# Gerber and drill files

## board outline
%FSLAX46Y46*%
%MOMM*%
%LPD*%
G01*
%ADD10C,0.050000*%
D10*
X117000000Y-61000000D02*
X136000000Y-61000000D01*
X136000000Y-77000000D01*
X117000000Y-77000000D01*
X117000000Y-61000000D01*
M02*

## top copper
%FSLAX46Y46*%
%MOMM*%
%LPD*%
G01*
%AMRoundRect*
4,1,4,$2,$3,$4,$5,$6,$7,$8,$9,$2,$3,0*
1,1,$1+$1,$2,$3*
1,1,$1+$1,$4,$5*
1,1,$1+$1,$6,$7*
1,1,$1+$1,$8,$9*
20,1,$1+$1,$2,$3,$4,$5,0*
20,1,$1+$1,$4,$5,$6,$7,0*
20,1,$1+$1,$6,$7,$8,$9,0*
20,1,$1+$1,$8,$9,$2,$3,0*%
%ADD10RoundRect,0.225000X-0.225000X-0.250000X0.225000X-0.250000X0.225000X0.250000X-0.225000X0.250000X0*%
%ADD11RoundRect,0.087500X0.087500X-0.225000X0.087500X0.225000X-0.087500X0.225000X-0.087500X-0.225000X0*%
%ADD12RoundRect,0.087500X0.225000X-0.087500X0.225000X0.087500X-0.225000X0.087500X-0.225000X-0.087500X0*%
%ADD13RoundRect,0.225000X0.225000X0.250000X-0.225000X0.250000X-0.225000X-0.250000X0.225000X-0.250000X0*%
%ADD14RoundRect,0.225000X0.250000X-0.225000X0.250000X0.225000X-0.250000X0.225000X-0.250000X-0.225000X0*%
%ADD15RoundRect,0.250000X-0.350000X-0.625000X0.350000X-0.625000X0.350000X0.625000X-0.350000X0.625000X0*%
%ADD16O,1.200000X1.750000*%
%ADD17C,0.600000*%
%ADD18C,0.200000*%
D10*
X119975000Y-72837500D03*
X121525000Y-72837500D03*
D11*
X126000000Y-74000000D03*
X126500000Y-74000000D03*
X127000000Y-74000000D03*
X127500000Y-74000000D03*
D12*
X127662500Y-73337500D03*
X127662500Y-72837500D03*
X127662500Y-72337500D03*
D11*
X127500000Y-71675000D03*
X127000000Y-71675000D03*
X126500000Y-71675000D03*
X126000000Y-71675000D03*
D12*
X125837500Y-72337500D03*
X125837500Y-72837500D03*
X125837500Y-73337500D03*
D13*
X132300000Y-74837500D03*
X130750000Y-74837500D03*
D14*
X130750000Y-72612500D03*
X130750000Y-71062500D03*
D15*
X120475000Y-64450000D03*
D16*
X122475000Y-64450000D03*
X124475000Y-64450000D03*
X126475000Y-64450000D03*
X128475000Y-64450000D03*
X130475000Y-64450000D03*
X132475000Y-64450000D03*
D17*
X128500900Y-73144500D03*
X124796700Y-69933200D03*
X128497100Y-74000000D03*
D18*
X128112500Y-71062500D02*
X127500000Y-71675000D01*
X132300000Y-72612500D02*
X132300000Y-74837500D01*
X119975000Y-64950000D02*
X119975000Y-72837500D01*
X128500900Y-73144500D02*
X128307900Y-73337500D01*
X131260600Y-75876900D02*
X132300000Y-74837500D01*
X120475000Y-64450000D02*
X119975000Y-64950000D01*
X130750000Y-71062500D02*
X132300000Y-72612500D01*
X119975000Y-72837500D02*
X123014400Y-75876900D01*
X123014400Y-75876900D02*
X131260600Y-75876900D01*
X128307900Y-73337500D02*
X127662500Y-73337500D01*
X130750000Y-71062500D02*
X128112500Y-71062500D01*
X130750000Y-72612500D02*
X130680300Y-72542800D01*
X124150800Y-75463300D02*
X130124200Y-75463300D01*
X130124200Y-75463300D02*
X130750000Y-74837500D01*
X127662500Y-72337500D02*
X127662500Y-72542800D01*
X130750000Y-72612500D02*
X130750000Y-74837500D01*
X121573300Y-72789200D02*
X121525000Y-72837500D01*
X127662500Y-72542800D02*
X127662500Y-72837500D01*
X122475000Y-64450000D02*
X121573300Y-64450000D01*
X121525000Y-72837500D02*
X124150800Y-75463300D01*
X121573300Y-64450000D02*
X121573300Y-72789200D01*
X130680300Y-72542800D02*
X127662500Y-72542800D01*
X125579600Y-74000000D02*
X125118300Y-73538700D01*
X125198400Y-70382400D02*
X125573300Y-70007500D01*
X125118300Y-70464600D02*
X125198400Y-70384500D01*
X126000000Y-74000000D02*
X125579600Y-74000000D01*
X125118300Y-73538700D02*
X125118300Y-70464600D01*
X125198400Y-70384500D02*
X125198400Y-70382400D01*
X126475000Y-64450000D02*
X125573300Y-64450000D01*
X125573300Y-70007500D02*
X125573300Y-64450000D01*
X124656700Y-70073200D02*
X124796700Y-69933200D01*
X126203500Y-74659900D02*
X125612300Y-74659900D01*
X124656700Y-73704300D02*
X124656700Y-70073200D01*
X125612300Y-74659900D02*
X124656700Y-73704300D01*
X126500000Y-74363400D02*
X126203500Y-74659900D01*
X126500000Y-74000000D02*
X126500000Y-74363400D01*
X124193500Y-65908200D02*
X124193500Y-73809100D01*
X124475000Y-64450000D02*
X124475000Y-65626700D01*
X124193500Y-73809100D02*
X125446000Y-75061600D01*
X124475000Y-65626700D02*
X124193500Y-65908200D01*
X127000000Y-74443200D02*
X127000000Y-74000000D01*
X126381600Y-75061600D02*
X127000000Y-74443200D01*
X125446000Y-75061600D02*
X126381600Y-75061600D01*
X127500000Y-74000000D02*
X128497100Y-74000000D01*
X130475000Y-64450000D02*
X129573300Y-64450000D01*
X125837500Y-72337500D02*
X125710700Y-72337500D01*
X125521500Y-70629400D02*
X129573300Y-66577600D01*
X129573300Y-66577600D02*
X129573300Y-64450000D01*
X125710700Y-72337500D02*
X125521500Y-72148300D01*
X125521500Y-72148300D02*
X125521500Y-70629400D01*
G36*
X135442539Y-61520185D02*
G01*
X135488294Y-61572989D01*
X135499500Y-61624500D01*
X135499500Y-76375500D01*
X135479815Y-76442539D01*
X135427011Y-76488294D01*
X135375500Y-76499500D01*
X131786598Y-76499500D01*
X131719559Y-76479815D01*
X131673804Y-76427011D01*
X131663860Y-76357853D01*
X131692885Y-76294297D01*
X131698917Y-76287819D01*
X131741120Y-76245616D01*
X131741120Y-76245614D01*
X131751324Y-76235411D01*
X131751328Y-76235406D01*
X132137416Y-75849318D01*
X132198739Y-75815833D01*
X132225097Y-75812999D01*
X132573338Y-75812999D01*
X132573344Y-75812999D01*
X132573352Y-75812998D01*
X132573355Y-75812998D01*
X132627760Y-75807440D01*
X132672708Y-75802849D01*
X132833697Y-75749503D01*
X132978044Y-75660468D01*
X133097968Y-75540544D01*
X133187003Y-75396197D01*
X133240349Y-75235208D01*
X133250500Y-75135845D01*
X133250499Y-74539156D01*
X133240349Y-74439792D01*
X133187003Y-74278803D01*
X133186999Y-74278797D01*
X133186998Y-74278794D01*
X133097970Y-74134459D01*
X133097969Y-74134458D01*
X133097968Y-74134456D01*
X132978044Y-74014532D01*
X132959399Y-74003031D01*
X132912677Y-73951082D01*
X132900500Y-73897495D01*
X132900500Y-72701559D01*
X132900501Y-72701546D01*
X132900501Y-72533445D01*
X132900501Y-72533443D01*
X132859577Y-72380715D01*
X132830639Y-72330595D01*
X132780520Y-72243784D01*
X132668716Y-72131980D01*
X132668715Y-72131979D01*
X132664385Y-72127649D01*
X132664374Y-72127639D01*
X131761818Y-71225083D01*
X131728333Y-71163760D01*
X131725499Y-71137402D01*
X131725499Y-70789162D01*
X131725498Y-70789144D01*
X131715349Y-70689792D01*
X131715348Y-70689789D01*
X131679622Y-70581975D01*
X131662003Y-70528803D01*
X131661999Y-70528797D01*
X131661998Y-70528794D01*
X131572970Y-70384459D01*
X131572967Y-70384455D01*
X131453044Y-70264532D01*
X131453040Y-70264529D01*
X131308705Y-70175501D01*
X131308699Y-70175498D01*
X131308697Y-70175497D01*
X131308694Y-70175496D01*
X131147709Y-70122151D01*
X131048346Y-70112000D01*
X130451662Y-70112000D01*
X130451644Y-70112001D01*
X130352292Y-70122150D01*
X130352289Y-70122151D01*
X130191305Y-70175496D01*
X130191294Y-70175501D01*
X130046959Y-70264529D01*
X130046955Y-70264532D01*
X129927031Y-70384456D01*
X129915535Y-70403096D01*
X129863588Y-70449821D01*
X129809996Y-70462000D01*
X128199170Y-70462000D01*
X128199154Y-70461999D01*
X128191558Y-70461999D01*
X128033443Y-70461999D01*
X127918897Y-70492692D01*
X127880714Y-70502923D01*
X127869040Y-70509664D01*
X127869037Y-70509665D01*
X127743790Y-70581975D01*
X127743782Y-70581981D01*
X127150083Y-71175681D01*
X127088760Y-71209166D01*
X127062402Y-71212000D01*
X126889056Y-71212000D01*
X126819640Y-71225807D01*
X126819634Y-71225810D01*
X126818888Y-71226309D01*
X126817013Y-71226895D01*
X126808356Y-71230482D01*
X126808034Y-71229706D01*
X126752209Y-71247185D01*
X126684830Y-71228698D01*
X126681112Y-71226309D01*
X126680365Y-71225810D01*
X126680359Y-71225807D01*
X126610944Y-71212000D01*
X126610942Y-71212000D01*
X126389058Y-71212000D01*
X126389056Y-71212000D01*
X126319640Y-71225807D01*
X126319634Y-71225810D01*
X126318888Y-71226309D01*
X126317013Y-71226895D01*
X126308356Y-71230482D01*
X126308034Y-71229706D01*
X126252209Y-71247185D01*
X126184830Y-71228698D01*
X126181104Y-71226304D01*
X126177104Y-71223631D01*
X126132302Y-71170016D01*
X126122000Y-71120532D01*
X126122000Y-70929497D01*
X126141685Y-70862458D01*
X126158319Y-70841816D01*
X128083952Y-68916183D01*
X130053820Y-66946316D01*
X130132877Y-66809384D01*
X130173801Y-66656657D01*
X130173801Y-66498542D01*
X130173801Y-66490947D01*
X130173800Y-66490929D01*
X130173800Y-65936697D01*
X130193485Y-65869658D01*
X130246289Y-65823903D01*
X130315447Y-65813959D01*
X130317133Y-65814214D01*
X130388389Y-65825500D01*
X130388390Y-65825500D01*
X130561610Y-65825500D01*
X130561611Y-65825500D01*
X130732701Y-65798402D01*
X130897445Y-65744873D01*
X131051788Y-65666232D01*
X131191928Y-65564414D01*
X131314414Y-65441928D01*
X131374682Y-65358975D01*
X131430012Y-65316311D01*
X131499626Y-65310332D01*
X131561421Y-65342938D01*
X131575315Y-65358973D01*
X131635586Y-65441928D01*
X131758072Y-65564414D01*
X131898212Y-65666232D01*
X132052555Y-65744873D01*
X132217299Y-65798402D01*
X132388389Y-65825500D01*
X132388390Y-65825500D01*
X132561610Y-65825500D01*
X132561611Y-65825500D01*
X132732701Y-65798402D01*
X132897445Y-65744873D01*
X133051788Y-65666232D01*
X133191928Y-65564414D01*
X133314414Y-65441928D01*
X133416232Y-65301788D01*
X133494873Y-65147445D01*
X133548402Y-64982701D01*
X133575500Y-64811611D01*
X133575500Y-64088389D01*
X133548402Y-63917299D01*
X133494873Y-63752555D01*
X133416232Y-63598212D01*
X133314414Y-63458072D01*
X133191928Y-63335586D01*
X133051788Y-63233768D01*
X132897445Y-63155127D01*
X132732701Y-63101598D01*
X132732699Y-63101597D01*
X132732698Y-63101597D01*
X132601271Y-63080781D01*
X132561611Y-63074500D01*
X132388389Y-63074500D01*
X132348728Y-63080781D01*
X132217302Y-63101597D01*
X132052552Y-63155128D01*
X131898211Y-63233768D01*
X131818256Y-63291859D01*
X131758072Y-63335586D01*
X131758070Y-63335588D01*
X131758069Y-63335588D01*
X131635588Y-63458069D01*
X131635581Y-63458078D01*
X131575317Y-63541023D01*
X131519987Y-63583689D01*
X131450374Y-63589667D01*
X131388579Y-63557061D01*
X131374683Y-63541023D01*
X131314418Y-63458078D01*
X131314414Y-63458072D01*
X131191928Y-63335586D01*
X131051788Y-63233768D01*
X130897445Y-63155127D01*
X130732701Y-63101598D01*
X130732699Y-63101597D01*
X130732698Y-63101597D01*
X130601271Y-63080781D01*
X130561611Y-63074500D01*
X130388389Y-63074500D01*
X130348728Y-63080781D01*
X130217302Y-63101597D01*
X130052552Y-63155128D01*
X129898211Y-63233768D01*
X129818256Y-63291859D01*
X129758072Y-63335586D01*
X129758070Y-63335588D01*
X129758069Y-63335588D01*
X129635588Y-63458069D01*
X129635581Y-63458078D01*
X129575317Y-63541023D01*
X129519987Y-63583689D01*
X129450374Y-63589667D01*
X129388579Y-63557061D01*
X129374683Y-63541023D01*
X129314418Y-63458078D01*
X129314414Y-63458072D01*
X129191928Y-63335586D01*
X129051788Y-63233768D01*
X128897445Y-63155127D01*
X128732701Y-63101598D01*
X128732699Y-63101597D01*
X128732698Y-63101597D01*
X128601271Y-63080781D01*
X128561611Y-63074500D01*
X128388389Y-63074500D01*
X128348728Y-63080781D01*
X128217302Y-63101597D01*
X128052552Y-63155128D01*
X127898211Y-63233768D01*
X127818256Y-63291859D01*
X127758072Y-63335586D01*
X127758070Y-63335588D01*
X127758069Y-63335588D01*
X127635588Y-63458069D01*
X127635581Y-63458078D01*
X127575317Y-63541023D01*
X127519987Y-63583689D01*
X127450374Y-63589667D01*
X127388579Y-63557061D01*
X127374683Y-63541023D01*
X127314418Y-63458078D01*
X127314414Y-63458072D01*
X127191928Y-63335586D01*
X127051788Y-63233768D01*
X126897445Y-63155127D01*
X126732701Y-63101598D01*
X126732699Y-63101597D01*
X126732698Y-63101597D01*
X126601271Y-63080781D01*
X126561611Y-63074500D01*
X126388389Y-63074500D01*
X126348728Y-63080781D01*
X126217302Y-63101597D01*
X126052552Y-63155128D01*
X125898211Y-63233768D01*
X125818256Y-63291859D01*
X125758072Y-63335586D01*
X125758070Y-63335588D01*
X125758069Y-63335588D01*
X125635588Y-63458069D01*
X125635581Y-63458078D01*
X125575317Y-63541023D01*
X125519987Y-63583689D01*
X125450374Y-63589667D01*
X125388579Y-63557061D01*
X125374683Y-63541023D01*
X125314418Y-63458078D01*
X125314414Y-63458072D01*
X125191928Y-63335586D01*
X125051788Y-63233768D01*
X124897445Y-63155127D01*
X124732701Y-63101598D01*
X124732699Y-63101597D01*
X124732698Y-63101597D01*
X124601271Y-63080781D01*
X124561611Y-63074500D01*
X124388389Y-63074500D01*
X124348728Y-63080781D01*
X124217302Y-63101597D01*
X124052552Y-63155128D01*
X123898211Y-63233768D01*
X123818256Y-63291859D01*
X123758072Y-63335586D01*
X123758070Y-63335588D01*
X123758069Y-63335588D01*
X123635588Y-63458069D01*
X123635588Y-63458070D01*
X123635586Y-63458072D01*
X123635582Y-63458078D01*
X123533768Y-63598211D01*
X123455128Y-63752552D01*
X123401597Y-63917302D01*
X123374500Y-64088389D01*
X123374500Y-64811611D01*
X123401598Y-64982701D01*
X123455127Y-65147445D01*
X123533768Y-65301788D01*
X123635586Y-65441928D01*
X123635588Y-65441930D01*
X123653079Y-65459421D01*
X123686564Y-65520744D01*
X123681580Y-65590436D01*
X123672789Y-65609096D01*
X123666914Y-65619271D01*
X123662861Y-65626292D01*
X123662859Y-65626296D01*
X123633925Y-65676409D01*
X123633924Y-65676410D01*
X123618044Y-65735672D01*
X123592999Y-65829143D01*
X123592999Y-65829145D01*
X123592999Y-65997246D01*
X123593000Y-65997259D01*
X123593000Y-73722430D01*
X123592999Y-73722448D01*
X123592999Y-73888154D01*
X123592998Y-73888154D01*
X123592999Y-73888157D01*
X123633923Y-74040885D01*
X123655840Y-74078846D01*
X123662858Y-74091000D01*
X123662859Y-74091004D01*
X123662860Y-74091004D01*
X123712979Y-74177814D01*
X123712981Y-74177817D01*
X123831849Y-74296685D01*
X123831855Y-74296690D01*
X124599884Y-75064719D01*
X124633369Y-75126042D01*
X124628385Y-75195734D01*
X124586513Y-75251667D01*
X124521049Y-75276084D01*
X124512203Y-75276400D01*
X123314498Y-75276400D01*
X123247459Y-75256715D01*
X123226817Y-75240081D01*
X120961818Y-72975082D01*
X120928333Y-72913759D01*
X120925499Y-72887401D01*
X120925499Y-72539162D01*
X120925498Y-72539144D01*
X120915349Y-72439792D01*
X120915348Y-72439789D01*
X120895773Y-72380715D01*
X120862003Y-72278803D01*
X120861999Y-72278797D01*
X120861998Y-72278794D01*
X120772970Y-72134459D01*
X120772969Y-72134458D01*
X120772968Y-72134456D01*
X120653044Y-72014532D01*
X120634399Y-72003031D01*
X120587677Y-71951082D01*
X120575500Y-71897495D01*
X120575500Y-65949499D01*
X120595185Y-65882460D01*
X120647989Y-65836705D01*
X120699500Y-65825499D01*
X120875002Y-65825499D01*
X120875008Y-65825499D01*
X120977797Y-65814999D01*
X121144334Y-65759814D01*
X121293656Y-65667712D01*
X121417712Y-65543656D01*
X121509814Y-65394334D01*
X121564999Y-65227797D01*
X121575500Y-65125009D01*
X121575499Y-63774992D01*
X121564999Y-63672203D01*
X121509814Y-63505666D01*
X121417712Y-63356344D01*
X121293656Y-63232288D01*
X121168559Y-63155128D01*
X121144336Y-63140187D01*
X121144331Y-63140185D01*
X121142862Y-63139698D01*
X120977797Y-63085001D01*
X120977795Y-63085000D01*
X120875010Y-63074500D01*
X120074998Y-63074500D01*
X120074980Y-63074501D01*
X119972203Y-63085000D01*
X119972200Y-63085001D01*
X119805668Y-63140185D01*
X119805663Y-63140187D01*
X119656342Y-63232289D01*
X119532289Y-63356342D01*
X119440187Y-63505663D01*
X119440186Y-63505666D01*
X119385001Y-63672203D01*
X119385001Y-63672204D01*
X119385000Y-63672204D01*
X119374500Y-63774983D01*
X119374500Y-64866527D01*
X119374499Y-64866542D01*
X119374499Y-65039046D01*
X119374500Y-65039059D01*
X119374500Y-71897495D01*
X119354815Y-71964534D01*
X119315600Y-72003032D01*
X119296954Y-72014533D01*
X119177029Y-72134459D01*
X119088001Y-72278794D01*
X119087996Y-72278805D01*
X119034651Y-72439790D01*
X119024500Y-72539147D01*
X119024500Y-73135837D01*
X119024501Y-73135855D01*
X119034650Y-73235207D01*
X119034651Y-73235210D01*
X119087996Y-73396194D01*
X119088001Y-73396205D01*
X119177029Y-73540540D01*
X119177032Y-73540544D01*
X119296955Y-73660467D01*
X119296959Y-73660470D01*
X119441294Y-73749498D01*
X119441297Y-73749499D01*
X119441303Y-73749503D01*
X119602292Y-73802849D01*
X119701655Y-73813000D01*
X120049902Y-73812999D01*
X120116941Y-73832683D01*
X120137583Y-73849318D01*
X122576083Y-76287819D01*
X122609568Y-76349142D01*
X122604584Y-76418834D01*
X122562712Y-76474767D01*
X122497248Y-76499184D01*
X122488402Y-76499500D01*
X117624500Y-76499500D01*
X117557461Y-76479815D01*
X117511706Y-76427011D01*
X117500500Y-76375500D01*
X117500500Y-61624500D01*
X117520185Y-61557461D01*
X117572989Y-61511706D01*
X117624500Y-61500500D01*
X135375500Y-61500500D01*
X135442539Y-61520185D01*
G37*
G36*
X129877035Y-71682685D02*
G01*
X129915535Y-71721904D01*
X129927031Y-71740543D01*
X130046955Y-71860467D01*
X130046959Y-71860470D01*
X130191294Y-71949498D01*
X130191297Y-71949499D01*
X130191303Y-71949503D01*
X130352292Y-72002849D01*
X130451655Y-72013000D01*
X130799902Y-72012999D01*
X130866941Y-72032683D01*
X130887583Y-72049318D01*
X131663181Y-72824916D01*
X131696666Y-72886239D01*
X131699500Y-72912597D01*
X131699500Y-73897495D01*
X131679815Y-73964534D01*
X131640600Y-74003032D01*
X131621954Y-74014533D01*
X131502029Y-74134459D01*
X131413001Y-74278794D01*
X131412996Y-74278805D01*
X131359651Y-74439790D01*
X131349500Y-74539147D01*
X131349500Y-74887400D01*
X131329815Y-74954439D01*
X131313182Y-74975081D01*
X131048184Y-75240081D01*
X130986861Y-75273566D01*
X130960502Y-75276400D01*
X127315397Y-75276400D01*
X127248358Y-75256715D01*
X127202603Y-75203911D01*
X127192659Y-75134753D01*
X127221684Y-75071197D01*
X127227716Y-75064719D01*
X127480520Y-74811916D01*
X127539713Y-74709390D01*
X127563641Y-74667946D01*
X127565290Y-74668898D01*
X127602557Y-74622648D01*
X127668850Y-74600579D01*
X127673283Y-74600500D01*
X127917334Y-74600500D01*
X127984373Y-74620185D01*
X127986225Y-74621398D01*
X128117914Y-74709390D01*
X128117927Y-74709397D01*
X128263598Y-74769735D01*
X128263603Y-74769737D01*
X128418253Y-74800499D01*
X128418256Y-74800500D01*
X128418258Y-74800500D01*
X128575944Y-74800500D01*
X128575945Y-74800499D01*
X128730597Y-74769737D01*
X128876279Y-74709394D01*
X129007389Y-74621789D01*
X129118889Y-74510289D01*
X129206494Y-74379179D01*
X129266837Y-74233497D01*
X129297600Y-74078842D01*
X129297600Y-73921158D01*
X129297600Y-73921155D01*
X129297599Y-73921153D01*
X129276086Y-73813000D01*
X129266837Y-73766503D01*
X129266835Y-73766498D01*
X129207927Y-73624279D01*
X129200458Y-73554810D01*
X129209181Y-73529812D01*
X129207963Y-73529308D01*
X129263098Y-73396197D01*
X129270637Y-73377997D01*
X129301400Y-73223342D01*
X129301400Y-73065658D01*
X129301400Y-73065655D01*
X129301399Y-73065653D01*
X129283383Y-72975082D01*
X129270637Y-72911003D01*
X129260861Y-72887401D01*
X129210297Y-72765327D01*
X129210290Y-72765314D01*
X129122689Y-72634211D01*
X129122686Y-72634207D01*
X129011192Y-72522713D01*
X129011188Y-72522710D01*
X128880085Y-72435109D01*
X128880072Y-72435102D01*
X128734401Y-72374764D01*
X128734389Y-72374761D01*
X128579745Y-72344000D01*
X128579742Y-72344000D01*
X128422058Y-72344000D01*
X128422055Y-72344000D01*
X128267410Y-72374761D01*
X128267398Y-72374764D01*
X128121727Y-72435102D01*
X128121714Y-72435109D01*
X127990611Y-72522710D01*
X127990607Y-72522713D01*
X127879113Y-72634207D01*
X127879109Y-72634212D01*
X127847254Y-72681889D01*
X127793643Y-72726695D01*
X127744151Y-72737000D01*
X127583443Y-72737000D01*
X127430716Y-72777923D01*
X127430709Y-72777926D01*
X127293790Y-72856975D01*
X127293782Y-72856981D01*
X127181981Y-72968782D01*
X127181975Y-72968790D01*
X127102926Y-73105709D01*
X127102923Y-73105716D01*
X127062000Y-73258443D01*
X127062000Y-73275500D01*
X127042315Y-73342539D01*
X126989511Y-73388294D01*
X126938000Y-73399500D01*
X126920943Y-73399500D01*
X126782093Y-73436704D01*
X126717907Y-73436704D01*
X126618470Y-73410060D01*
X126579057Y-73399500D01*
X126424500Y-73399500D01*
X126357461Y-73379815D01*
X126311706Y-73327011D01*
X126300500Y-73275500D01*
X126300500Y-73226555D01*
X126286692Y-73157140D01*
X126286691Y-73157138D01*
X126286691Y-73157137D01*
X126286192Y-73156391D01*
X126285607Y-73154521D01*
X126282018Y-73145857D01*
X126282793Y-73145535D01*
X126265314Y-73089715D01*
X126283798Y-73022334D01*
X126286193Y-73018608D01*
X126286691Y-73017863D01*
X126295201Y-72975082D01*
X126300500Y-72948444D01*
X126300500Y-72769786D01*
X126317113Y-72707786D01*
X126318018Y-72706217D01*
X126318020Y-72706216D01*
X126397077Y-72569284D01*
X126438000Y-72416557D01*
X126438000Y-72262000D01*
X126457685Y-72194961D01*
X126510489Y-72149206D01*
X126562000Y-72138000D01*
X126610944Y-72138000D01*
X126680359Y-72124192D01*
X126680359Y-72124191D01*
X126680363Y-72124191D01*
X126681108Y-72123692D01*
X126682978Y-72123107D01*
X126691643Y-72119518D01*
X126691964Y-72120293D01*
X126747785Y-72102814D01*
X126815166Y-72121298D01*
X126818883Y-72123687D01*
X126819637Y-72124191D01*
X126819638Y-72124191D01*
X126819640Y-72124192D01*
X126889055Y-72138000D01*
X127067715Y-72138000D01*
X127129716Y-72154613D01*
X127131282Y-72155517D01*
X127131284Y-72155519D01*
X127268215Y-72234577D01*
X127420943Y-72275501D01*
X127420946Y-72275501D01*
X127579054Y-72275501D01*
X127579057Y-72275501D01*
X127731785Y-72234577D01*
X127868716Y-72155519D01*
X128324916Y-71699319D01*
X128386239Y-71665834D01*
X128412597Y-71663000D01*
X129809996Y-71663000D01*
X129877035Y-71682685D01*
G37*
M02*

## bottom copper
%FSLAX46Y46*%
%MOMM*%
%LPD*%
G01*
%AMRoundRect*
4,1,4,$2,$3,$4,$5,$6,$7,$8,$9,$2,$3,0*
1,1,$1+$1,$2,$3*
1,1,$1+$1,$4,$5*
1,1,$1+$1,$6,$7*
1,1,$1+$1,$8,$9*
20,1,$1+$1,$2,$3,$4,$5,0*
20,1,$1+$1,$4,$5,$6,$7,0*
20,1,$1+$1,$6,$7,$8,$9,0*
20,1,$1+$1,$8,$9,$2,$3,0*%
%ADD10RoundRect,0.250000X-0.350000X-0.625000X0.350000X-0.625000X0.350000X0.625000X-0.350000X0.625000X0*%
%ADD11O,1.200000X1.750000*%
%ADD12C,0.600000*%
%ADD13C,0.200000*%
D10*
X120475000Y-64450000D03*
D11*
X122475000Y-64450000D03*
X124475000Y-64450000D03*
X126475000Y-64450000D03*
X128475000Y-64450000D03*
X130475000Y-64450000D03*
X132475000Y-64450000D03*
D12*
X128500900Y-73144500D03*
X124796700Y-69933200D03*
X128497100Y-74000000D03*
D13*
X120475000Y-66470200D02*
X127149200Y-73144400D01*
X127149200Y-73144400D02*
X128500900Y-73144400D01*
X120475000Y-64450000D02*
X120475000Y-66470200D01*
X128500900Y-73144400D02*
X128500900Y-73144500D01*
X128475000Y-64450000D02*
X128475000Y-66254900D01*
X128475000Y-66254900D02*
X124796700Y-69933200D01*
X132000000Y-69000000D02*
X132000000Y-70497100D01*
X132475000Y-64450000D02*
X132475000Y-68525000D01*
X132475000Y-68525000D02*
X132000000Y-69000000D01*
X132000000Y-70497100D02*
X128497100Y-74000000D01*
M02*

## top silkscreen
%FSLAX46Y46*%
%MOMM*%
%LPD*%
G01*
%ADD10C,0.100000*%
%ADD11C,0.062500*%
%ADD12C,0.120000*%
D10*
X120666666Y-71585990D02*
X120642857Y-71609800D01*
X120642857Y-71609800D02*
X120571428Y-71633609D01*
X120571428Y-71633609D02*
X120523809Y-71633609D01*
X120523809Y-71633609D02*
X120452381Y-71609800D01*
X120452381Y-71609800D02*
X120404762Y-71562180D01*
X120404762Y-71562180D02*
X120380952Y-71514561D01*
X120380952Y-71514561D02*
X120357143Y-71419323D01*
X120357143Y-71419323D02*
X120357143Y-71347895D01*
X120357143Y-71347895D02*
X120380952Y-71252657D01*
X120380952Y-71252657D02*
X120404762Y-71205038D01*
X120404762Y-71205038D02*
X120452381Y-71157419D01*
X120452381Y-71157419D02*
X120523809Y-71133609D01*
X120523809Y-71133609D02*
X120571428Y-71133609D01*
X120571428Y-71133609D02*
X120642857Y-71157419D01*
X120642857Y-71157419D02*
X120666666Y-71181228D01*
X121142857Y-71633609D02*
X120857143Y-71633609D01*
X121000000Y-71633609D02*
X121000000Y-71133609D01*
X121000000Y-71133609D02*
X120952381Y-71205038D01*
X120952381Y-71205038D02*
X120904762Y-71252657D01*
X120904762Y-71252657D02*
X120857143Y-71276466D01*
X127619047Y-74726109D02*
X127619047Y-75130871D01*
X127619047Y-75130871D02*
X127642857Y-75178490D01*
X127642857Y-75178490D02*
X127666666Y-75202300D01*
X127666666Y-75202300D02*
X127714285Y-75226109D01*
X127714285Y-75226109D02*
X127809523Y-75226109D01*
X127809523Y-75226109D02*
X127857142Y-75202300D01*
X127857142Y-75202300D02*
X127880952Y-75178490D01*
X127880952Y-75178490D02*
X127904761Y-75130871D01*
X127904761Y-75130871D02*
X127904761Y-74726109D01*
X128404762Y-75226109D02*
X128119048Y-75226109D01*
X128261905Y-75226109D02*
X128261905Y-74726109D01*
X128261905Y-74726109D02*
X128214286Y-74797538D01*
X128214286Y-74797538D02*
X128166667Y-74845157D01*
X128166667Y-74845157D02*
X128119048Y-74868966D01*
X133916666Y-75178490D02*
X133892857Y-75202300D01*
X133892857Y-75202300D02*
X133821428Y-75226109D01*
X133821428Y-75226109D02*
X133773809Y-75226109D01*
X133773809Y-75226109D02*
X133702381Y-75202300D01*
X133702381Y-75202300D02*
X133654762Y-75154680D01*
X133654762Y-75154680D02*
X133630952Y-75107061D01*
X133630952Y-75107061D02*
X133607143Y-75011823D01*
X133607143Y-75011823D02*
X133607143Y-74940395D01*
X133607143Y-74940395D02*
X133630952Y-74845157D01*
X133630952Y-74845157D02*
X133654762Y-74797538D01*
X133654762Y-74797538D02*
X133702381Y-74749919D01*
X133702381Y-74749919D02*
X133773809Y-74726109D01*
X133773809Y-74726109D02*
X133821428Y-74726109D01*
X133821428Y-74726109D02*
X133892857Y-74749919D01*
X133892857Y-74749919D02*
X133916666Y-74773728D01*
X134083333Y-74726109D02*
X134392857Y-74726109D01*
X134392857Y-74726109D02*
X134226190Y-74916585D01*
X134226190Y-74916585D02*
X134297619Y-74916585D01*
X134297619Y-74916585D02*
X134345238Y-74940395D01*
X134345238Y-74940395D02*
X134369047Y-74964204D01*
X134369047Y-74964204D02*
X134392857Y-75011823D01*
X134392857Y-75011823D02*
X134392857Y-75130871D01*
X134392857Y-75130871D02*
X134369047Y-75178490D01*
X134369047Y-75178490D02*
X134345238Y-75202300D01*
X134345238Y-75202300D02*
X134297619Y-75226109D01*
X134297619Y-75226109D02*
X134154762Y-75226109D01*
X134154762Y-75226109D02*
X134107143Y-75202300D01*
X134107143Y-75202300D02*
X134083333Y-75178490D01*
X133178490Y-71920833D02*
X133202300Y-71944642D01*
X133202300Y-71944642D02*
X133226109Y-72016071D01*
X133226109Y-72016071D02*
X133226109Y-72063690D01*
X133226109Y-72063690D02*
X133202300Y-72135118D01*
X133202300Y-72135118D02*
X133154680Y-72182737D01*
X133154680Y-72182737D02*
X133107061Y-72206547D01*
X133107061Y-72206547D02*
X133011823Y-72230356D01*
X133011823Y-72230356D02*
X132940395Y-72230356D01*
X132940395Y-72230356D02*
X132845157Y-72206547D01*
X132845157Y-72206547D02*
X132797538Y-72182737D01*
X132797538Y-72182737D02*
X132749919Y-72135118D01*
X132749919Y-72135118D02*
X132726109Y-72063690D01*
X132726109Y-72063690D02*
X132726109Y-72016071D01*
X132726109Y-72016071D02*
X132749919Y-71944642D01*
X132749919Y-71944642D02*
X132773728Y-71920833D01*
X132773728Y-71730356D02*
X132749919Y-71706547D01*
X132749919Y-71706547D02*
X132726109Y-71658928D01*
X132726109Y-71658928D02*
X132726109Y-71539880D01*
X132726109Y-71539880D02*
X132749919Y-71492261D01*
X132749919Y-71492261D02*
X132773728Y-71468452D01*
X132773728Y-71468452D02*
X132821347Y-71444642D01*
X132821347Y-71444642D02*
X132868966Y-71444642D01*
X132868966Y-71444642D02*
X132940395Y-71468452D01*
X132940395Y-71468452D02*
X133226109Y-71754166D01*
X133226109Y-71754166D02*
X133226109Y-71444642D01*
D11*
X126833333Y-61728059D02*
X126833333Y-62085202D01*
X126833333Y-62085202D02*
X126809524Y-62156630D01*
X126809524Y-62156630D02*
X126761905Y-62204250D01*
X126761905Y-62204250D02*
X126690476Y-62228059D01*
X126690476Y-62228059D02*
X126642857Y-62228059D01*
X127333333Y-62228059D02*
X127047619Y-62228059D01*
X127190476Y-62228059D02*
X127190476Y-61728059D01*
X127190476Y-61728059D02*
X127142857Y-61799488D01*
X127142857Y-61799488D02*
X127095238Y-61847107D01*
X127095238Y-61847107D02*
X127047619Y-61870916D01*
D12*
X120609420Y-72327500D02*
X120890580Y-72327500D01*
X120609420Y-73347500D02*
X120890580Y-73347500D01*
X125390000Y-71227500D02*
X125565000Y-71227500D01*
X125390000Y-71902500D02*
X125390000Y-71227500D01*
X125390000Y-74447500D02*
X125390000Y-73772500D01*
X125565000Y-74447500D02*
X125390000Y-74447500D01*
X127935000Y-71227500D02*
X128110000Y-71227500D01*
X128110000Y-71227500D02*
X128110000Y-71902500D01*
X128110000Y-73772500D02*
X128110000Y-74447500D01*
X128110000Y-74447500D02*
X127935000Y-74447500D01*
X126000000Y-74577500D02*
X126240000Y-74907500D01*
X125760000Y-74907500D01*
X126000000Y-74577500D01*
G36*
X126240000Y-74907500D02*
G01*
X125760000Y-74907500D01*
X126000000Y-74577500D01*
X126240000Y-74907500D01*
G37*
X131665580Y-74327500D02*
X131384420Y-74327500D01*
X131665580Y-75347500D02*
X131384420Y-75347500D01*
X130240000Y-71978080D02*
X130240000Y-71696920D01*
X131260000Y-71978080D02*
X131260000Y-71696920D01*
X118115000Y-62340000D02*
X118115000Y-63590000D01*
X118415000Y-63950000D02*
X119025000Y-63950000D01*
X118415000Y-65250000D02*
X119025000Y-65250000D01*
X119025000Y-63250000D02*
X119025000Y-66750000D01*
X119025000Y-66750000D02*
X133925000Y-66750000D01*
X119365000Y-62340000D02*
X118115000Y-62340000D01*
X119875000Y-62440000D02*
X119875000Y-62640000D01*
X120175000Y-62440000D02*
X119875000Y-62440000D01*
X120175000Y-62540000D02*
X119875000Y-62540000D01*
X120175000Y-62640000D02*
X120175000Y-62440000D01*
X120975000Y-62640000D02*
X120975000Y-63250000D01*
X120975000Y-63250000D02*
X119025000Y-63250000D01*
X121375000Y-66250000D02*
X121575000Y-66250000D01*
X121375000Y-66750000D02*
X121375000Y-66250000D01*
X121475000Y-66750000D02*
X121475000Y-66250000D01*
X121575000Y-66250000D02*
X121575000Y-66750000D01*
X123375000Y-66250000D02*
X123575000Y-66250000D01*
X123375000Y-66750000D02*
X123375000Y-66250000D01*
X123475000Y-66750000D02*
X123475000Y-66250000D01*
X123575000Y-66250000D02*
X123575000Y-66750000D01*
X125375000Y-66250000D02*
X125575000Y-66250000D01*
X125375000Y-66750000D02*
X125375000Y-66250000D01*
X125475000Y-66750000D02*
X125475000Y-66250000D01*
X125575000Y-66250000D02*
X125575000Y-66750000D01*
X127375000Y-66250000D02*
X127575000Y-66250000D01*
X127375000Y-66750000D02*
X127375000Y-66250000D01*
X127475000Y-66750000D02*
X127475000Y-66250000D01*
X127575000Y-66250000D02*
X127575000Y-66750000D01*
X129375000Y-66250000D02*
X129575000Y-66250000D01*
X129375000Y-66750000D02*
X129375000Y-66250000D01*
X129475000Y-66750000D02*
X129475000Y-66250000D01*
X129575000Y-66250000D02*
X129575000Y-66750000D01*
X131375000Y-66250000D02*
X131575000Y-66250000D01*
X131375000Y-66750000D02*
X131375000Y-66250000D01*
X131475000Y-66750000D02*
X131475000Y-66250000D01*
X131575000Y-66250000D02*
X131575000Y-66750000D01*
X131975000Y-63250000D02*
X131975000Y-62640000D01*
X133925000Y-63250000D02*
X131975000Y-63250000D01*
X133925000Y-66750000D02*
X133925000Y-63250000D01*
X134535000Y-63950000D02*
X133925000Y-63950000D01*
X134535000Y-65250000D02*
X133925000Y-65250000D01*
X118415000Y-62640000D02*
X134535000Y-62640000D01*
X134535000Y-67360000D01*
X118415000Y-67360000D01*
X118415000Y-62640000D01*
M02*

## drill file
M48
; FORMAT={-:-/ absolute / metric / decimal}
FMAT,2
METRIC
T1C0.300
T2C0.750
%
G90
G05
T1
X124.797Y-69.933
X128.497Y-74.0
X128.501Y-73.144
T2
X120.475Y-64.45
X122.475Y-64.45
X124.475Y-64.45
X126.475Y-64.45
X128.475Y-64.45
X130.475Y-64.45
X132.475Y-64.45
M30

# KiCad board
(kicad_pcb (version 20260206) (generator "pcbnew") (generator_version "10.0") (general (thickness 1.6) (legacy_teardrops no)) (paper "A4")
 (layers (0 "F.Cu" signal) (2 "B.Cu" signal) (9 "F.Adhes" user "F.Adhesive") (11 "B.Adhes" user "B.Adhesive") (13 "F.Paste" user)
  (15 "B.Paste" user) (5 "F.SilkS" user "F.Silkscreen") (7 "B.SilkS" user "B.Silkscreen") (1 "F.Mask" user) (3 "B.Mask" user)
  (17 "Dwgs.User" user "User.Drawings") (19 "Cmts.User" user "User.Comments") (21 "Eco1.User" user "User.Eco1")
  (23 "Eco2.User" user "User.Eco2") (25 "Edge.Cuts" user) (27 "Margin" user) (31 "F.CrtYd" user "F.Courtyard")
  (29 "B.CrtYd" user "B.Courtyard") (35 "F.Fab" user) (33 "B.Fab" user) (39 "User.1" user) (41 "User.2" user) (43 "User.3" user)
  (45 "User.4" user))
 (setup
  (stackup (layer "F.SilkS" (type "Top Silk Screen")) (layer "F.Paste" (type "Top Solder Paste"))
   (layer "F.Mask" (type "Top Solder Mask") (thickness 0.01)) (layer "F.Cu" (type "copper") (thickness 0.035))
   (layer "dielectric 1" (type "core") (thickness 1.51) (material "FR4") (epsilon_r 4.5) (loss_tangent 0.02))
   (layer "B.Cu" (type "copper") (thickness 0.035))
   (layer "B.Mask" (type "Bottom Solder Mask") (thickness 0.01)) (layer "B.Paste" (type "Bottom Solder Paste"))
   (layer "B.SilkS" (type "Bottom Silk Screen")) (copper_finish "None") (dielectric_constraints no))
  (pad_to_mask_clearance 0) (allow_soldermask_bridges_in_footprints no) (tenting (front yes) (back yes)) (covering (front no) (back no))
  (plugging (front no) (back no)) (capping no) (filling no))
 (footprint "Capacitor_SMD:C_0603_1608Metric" (layer "F.Cu") (at 120.75 72.8375)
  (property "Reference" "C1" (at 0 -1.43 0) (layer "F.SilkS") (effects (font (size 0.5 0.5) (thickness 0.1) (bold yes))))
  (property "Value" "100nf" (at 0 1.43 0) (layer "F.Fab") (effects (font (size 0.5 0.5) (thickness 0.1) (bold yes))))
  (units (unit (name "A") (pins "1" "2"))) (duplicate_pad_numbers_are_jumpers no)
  (fp_line (start -0.14058 -0.51) (end 0.14058 -0.51) (stroke (width 0.12) (type solid)) (layer "F.SilkS"))
  (fp_line (start -0.14058 0.51) (end 0.14058 0.51) (stroke (width 0.12) (type solid)) (layer "F.SilkS"))
  (pad "1" smd roundrect (at -0.775 0) (size 0.9 0.95) (layers "F.Cu" "F.Mask" "F.Paste") (roundrect_rratio 0.25) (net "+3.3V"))
  (pad "2" smd roundrect (at 0.775 0) (size 0.9 0.95) (layers "F.Cu" "F.Mask" "F.Paste") (roundrect_rratio 0.25) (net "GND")))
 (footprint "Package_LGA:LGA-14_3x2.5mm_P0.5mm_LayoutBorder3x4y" (layer "F.Cu") (at 126.75 72.8375 90)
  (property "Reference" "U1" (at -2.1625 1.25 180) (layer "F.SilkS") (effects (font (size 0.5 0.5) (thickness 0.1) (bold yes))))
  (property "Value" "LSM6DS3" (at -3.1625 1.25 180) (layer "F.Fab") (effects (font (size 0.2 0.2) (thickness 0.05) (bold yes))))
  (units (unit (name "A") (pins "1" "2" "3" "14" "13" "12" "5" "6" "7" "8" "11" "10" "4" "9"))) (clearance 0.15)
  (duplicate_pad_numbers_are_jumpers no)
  (fp_line (start 1.61 -1.36) (end 1.61 -1.185) (stroke (width 0.12) (type solid)) (layer "F.SilkS"))
  (fp_line (start 0.935 -1.36) (end 1.61 -1.36) (stroke (width 0.12) (type solid)) (layer "F.SilkS"))
  (fp_line (start -1.61 -1.36) (end -0.935 -1.36) (stroke (width 0.12) (type solid)) (layer "F.SilkS"))
  (fp_line (start -1.61 -1.185) (end -1.61 -1.36) (stroke (width 0.12) (type solid)) (layer "F.SilkS"))
  (fp_line (start 1.61 1.185) (end 1.61 1.36) (stroke (width 0.12) (type solid)) (layer "F.SilkS"))
  (fp_line (start 1.61 1.36) (end 0.935 1.36) (stroke (width 0.12) (type solid)) (layer "F.SilkS"))
  (fp_line (start -0.935 1.36) (end -1.61 1.36) (stroke (width 0.12) (type solid)) (layer "F.SilkS"))
  (fp_line (start -1.61 1.36) (end -1.61 1.185) (stroke (width 0.12) (type solid)) (layer "F.SilkS"))
  (fp_poly (pts (xy -1.74 -0.75) (xy -2.07 -0.51) (xy -2.07 -0.99)) (stroke (width 0.12) (type solid)) (fill yes) (layer "F.SilkS"))
  (pad "1" smd roundrect (at -1.1625 -0.75 90) (size 0.625 0.35) (layers "F.Cu" "F.Mask" "F.Paste") (roundrect_rratio 0.25)
   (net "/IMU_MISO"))
  (pad "2" smd roundrect (at -1.1625 -0.25 90) (size 0.625 0.35) (layers "F.Cu" "F.Mask" "F.Paste") (roundrect_rratio 0.25)
   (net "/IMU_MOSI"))
  (pad "3" smd roundrect (at -1.1625 0.25 90) (size 0.625 0.35) (layers "F.Cu" "F.Mask" "F.Paste") (roundrect_rratio 0.25) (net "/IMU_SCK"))
  (pad "4" smd roundrect (at -1.1625 0.75 90) (size 0.625 0.35) (layers "F.Cu" "F.Mask" "F.Paste") (roundrect_rratio 0.25) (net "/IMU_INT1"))
  (pad "5" smd roundrect (at -0.5 0.9125 90) (size 0.35 0.625) (layers "F.Cu" "F.Mask" "F.Paste") (roundrect_rratio 0.25) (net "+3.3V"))
  (pad "6" smd roundrect (at 0 0.9125 90) (size 0.35 0.625) (layers "F.Cu" "F.Mask" "F.Paste") (roundrect_rratio 0.25) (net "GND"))
  (pad "7" smd roundrect (at 0.5 0.9125 90) (size 0.35 0.625) (layers "F.Cu" "F.Mask" "F.Paste") (roundrect_rratio 0.25) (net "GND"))
  (pad "8" smd roundrect (at 1.1625 0.75 90) (size 0.625 0.35) (layers "F.Cu" "F.Mask" "F.Paste") (roundrect_rratio 0.25) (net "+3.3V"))
  (pad "9" smd roundrect (at 1.1625 0.25 90) (size 0.625 0.35) (layers "F.Cu" "F.Mask" "F.Paste") (roundrect_rratio 0.25)
   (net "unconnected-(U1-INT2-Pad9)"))
  (pad "10" smd roundrect (at 1.1625 -0.25 90) (size 0.625 0.35) (layers "F.Cu" "F.Mask" "F.Paste") (roundrect_rratio 0.25)
   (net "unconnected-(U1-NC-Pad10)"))
  (pad "11" smd roundrect (at 1.1625 -0.75 90) (size 0.625 0.35) (layers "F.Cu" "F.Mask" "F.Paste") (roundrect_rratio 0.25)
   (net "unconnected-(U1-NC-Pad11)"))
  (pad "12" smd roundrect (at 0.5 -0.9125 90) (size 0.35 0.625) (layers "F.Cu" "F.Mask" "F.Paste") (roundrect_rratio 0.25) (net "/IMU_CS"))
  (pad "13" smd roundrect (at 0 -0.9125 90) (size 0.35 0.625) (layers "F.Cu" "F.Mask" "F.Paste") (roundrect_rratio 0.25)
   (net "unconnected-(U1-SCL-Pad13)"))
  (pad "14" smd roundrect (at -0.5 -0.9125 90) (size 0.35 0.625) (layers "F.Cu" "F.Mask" "F.Paste") (roundrect_rratio 0.25)
   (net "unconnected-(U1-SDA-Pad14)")))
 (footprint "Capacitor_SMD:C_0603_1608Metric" (layer "F.Cu") (at 131.525 74.8375 180)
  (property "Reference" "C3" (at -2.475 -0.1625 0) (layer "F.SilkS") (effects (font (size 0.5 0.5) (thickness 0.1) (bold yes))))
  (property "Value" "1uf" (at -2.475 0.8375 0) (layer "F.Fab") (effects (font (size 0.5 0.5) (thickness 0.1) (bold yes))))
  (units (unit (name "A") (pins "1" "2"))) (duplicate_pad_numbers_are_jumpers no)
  (fp_line (start -0.14058 0.51) (end 0.14058 0.51) (stroke (width 0.12) (type solid)) (layer "F.SilkS"))
  (fp_line (start -0.14058 -0.51) (end 0.14058 -0.51) (stroke (width 0.12) (type solid)) (layer "F.SilkS"))
  (pad "1" smd roundrect (at -0.775 0 180) (size 0.9 0.95) (layers "F.Cu" "F.Mask" "F.Paste") (roundrect_rratio 0.25) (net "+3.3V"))
  (pad "2" smd roundrect (at 0.775 0 180) (size 0.9 0.95) (layers "F.Cu" "F.Mask" "F.Paste") (roundrect_rratio 0.25) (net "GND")))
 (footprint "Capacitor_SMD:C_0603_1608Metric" (layer "F.Cu") (at 130.75 71.8375 90)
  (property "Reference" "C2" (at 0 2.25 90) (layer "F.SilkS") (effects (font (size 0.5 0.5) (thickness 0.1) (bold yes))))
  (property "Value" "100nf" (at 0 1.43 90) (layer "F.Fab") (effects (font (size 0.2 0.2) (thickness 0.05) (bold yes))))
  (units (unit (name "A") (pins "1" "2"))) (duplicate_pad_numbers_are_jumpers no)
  (fp_line (start -0.14058 -0.51) (end 0.14058 -0.51) (stroke (width 0.12) (type solid)) (layer "F.SilkS"))
  (fp_line (start -0.14058 0.51) (end 0.14058 0.51) (stroke (width 0.12) (type solid)) (layer "F.SilkS"))
  (pad "1" smd roundrect (at -0.775 0 90) (size 0.9 0.95) (layers "F.Cu" "F.Mask" "F.Paste") (roundrect_rratio 0.25) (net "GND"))
  (pad "2" smd roundrect (at 0.775 0 90) (size 0.9 0.95) (layers "F.Cu" "F.Mask" "F.Paste") (roundrect_rratio 0.25) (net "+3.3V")))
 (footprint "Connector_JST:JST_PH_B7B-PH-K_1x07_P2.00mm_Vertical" (layer "F.Cu") (at 120.475 64.45)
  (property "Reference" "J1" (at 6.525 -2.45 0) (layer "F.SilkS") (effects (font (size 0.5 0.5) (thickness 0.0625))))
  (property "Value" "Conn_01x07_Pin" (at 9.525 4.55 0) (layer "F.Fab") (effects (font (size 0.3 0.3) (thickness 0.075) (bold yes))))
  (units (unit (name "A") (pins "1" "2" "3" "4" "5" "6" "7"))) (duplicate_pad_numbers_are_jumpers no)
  (fp_line (start -2.36 -2.11) (end -2.36 -0.86) (stroke (width 0.12) (type solid)) (layer "F.SilkS"))
  (fp_line (start -2.06 -0.5) (end -1.45 -0.5) (stroke (width 0.12) (type solid)) (layer "F.SilkS"))
  (fp_line (start -2.06 0.8) (end -1.45 0.8) (stroke (width 0.12) (type solid)) (layer "F.SilkS"))
  (fp_line (start -1.45 -1.2) (end -1.45 2.3) (stroke (width 0.12) (type solid)) (layer "F.SilkS"))
  (fp_line (start -1.45 2.3) (end 13.45 2.3) (stroke (width 0.12) (type solid)) (layer "F.SilkS"))
  (fp_line (start -1.11 -2.11) (end -2.36 -2.11) (stroke (width 0.12) (type solid)) (layer "F.SilkS"))
  (fp_line (start -0.6 -2.01) (end -0.6 -1.81) (stroke (width 0.12) (type solid)) (layer "F.SilkS"))
  (fp_line (start -0.3 -2.01) (end -0.6 -2.01) (stroke (width 0.12) (type solid)) (layer "F.SilkS"))
  (fp_line (start -0.3 -1.91) (end -0.6 -1.91) (stroke (width 0.12) (type solid)) (layer "F.SilkS"))
  (fp_line (start -0.3 -1.81) (end -0.3 -2.01) (stroke (width 0.12) (type solid)) (layer "F.SilkS"))
  (fp_line (start 0.5 -1.81) (end 0.5 -1.2) (stroke (width 0.12) (type solid)) (layer "F.SilkS"))
  (fp_line (start 0.5 -1.2) (end -1.45 -1.2) (stroke (width 0.12) (type solid)) (layer "F.SilkS"))
  (fp_line (start 0.9 1.8) (end 1.1 1.8) (stroke (width 0.12) (type solid)) (layer "F.SilkS"))
  (fp_line (start 0.9 2.3) (end 0.9 1.8) (stroke (width 0.12) (type solid)) (layer "F.SilkS"))
  (fp_line (start 1 2.3) (end 1 1.8) (stroke (width 0.12) (type solid)) (layer "F.SilkS"))
  (fp_line (start 1.1 1.8) (end 1.1 2.3) (stroke (width 0.12) (type solid)) (layer "F.SilkS"))
  (fp_line (start 2.9 1.8) (end 3.1 1.8) (stroke (width 0.12) (type solid)) (layer "F.SilkS"))
  (fp_line (start 2.9 2.3) (end 2.9 1.8) (stroke (width 0.12) (type solid)) (layer "F.SilkS"))
  (fp_line (start 3 2.3) (end 3 1.8) (stroke (width 0.12) (type solid)) (layer "F.SilkS"))
  (fp_line (start 3.1 1.8) (end 3.1 2.3) (stroke (width 0.12) (type solid)) (layer "F.SilkS"))
  (fp_line (start 4.9 1.8) (end 5.1 1.8) (stroke (width 0.12) (type solid)) (layer "F.SilkS"))
  (fp_line (start 4.9 2.3) (end 4.9 1.8) (stroke (width 0.12) (type solid)) (layer "F.SilkS"))
  (fp_line (start 5 2.3) (end 5 1.8) (stroke (width 0.12) (type solid)) (layer "F.SilkS"))
  (fp_line (start 5.1 1.8) (end 5.1 2.3) (stroke (width 0.12) (type solid)) (layer "F.SilkS"))
  (fp_line (start 6.9 1.8) (end 7.1 1.8) (stroke (width 0.12) (type solid)) (layer "F.SilkS"))
  (fp_line (start 6.9 2.3) (end 6.9 1.8) (stroke (width 0.12) (type solid)) (layer "F.SilkS"))
  (fp_line (start 7 2.3) (end 7 1.8) (stroke (width 0.12) (type solid)) (layer "F.SilkS"))
  (fp_line (start 7.1 1.8) (end 7.1 2.3) (stroke (width 0.12) (type solid)) (layer "F.SilkS"))
  (fp_line (start 8.9 1.8) (end 9.1 1.8) (stroke (width 0.12) (type solid)) (layer "F.SilkS"))
  (fp_line (start 8.9 2.3) (end 8.9 1.8) (stroke (width 0.12) (type solid)) (layer "F.SilkS"))
  (fp_line (start 9 2.3) (end 9 1.8) (stroke (width 0.12) (type solid)) (layer "F.SilkS"))
  (fp_line (start 9.1 1.8) (end 9.1 2.3) (stroke (width 0.12) (type solid)) (layer "F.SilkS"))
  (fp_line (start 10.9 1.8) (end 11.1 1.8) (stroke (width 0.12) (type solid)) (layer "F.SilkS"))
  (fp_line (start 10.9 2.3) (end 10.9 1.8) (stroke (width 0.12) (type solid)) (layer "F.SilkS"))
  (fp_line (start 11 2.3) (end 11 1.8) (stroke (width 0.12) (type solid)) (layer "F.SilkS"))
  (fp_line (start 11.1 1.8) (end 11.1 2.3) (stroke (width 0.12) (type solid)) (layer "F.SilkS"))
  (fp_line (start 11.5 -1.2) (end 11.5 -1.81) (stroke (width 0.12) (type solid)) (layer "F.SilkS"))
  (fp_line (start 13.45 -1.2) (end 11.5 -1.2) (stroke (width 0.12) (type solid)) (layer "F.SilkS"))
  (fp_line (start 13.45 2.3) (end 13.45 -1.2) (stroke (width 0.12) (type solid)) (layer "F.SilkS"))
  (fp_line (start 14.06 -0.5) (end 13.45 -0.5) (stroke (width 0.12) (type solid)) (layer "F.SilkS"))
  (fp_line (start 14.06 0.8) (end 13.45 0.8) (stroke (width 0.12) (type solid)) (layer "F.SilkS"))
  (fp_rect (start -2.06 -1.81) (end 14.06 2.91) (stroke (width 0.12) (type solid)) (fill no) (layer "F.SilkS"))
  (pad "1" thru_hole roundrect (at 0 0) (size 1.2 1.75) (drill 0.75) (layers "*.Cu" "*.Mask") (remove_unused_layers no)
   (roundrect_rratio 0.208333) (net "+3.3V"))
  (pad "2" thru_hole oval (at 2 0) (size 1.2 1.75) (drill 0.75) (layers "*.Cu" "*.Mask") (remove_unused_layers no) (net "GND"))
  (pad "3" thru_hole oval (at 4 0) (size 1.2 1.75) (drill 0.75) (layers "*.Cu" "*.Mask") (remove_unused_layers no) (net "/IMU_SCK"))
  (pad "4" thru_hole oval (at 6 0) (size 1.2 1.75) (drill 0.75) (layers "*.Cu" "*.Mask") (remove_unused_layers no) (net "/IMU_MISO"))
  (pad "5" thru_hole oval (at 8 0) (size 1.2 1.75) (drill 0.75) (layers "*.Cu" "*.Mask") (remove_unused_layers no) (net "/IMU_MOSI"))
  (pad "6" thru_hole oval (at 10 0) (size 1.2 1.75) (drill 0.75) (layers "*.Cu" "*.Mask") (remove_unused_layers no) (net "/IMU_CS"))
  (pad "7" thru_hole oval (at 12 0) (size 1.2 1.75) (drill 0.75) (layers "*.Cu" "*.Mask") (remove_unused_layers no) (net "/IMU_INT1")))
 (gr_rect (start 117 61) (end 136 77) (stroke (width 0.05) (type default)) (fill no) (layer "Edge.Cuts"))
 (segment (start 128.1125 71.0625) (end 127.5 71.675) (width 0.2) (layer "F.Cu") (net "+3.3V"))
 (segment (start 132.3 72.6125) (end 132.3 74.8375) (width 0.2) (layer "F.Cu") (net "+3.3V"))
 (segment (start 119.975 64.95) (end 119.975 72.8375) (width 0.2) (layer "F.Cu") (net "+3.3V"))
 (segment (start 128.5009 73.1445) (end 128.3079 73.3375) (width 0.2) (layer "F.Cu") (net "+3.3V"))
 (segment (start 131.2606 75.8769) (end 132.3 74.8375) (width 0.2) (layer "F.Cu") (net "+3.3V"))
 (segment (start 120.475 64.45) (end 119.975 64.95) (width 0.2) (layer "F.Cu") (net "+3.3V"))
 (segment (start 130.75 71.0625) (end 132.3 72.6125) (width 0.2) (layer "F.Cu") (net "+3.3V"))
 (segment (start 119.975 72.8375) (end 123.0144 75.8769) (width 0.2) (layer "F.Cu") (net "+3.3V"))
 (segment (start 123.0144 75.8769) (end 131.2606 75.8769) (width 0.2) (layer "F.Cu") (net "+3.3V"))
 (segment (start 128.3079 73.3375) (end 127.6625 73.3375) (width 0.2) (layer "F.Cu") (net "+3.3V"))
 (segment (start 130.75 71.0625) (end 128.1125 71.0625) (width 0.2) (layer "F.Cu") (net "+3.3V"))
 (via (at 128.5009 73.1445) (size 0.6) (drill 0.3) (layers "F.Cu" "B.Cu") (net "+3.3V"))
 (segment (start 120.475 66.4702) (end 127.1492 73.1444) (width 0.2) (layer "B.Cu") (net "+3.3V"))
 (segment (start 127.1492 73.1444) (end 128.5009 73.1444) (width 0.2) (layer "B.Cu") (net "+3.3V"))
 (segment (start 120.475 64.45) (end 120.475 66.4702) (width 0.2) (layer "B.Cu") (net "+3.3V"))
 (segment (start 128.5009 73.1444) (end 128.5009 73.1445) (width 0.2) (layer "B.Cu") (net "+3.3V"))
 (segment (start 130.75 72.6125) (end 130.6803 72.5428) (width 0.2) (layer "F.Cu") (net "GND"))
 (segment (start 124.1508 75.4633) (end 130.1242 75.4633) (width 0.2) (layer "F.Cu") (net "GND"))
 (segment (start 130.1242 75.4633) (end 130.75 74.8375) (width 0.2) (layer "F.Cu") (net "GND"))
 (segment (start 127.6625 72.3375) (end 127.6625 72.5428) (width 0.2) (layer "F.Cu") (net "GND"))
 (segment (start 130.75 72.6125) (end 130.75 74.8375) (width 0.2) (layer "F.Cu") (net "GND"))
 (segment (start 121.5733 72.7892) (end 121.525 72.8375) (width 0.2) (layer "F.Cu") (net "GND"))
 (segment (start 127.6625 72.5428) (end 127.6625 72.8375) (width 0.2) (layer "F.Cu") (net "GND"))
 (segment (start 122.475 64.45) (end 121.5733 64.45) (width 0.2) (layer "F.Cu") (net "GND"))
 (segment (start 121.525 72.8375) (end 124.1508 75.4633) (width 0.2) (layer "F.Cu") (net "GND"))
 (segment (start 121.5733 64.45) (end 121.5733 72.7892) (width 0.2) (layer "F.Cu") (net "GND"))
 (segment (start 130.6803 72.5428) (end 127.6625 72.5428) (width 0.2) (layer "F.Cu") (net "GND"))
 (segment (start 125.5796 74) (end 125.1183 73.5387) (width 0.2) (layer "F.Cu") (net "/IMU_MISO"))
 (segment (start 125.1984 70.3824) (end 125.5733 70.0075) (width 0.2) (layer "F.Cu") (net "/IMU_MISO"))
 (segment (start 125.1183 70.4646) (end 125.1984 70.3845) (width 0.2) (layer "F.Cu") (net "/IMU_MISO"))
 (segment (start 126 74) (end 125.5796 74) (width 0.2) (layer "F.Cu") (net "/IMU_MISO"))
 (segment (start 125.1183 73.5387) (end 125.1183 70.4646) (width 0.2) (layer "F.Cu") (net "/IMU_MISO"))
 (segment (start 125.1984 70.3845) (end 125.1984 70.3824) (width 0.2) (layer "F.Cu") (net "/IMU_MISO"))
 (segment (start 126.475 64.45) (end 125.5733 64.45) (width 0.2) (layer "F.Cu") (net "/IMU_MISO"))
 (segment (start 125.5733 70.0075) (end 125.5733 64.45) (width 0.2) (layer "F.Cu") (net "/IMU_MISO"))
 (segment (start 124.6567 70.0732) (end 124.7967 69.9332) (width 0.2) (layer "F.Cu") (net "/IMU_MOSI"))
 (segment (start 126.2035 74.6599) (end 125.6123 74.6599) (width 0.2) (layer "F.Cu") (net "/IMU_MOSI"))
 (segment (start 124.6567 73.7043) (end 124.6567 70.0732) (width 0.2) (layer "F.Cu") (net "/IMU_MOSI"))
 (segment (start 125.6123 74.6599) (end 124.6567 73.7043) (width 0.2) (layer "F.Cu") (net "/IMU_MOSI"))
 (segment (start 126.5 74.3634) (end 126.2035 74.6599) (width 0.2) (layer "F.Cu") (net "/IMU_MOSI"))
 (segment (start 126.5 74) (end 126.5 74.3634) (width 0.2) (layer "F.Cu") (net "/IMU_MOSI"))
 (via (at 124.7967 69.9332) (size 0.6) (drill 0.3) (layers "F.Cu" "B.Cu") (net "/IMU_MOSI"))
 (segment (start 128.475 64.45) (end 128.475 66.2549) (width 0.2) (layer "B.Cu") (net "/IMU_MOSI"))
 (segment (start 128.475 66.2549) (end 124.7967 69.9332) (width 0.2) (layer "B.Cu") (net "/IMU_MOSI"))
 (segment (start 124.1935 65.9082) (end 124.1935 73.8091) (width 0.2) (layer "F.Cu") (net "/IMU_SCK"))
 (segment (start 124.475 64.45) (end 124.475 65.6267) (width 0.2) (layer "F.Cu") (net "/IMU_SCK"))
 (segment (start 124.1935 73.8091) (end 125.446 75.0616) (width 0.2) (layer "F.Cu") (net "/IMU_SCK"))
 (segment (start 124.475 65.6267) (end 124.1935 65.9082) (width 0.2) (layer "F.Cu") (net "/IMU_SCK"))
 (segment (start 127 74.4432) (end 127 74) (width 0.2) (layer "F.Cu") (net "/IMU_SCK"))
 (segment (start 126.3816 75.0616) (end 127 74.4432) (width 0.2) (layer "F.Cu") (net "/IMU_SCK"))
 (segment (start 125.446 75.0616) (end 126.3816 75.0616) (width 0.2) (layer "F.Cu") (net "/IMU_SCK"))
 (segment (start 127.5 74) (end 128.4971 74) (width 0.2) (layer "F.Cu") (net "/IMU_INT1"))
 (via (at 128.4971 74) (size 0.6) (drill 0.3) (layers "F.Cu" "B.Cu") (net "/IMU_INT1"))
 (segment (start 132 69) (end 132 70.4971) (width 0.2) (layer "B.Cu") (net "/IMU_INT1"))
 (segment (start 132.475 64.45) (end 132.475 68.525) (width 0.2) (layer "B.Cu") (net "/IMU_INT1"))
 (segment (start 132.475 68.525) (end 132 69) (width 0.2) (layer "B.Cu") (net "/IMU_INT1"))
 (segment (start 132 70.4971) (end 128.4971 74) (width 0.2) (layer "B.Cu") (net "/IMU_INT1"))
 (segment (start 130.475 64.45) (end 129.5733 64.45) (width 0.2) (layer "F.Cu") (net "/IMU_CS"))
 (segment (start 125.8375 72.3375) (end 125.7107 72.3375) (width 0.2) (layer "F.Cu") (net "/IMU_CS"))
 (segment (start 125.5215 70.6294) (end 129.5733 66.5776) (width 0.2) (layer "F.Cu") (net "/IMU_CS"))
 (segment (start 129.5733 66.5776) (end 129.5733 64.45) (width 0.2) (layer "F.Cu") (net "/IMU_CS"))
 (segment (start 125.7107 72.3375) (end 125.5215 72.1483) (width 0.2) (layer "F.Cu") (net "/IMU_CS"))
 (segment (start 125.5215 72.1483) (end 125.5215 70.6294) (width 0.2) (layer "F.Cu") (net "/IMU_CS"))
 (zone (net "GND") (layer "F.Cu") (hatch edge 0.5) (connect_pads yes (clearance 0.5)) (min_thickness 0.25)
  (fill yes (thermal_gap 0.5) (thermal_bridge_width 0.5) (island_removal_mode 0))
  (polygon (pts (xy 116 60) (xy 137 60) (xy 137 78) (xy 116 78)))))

